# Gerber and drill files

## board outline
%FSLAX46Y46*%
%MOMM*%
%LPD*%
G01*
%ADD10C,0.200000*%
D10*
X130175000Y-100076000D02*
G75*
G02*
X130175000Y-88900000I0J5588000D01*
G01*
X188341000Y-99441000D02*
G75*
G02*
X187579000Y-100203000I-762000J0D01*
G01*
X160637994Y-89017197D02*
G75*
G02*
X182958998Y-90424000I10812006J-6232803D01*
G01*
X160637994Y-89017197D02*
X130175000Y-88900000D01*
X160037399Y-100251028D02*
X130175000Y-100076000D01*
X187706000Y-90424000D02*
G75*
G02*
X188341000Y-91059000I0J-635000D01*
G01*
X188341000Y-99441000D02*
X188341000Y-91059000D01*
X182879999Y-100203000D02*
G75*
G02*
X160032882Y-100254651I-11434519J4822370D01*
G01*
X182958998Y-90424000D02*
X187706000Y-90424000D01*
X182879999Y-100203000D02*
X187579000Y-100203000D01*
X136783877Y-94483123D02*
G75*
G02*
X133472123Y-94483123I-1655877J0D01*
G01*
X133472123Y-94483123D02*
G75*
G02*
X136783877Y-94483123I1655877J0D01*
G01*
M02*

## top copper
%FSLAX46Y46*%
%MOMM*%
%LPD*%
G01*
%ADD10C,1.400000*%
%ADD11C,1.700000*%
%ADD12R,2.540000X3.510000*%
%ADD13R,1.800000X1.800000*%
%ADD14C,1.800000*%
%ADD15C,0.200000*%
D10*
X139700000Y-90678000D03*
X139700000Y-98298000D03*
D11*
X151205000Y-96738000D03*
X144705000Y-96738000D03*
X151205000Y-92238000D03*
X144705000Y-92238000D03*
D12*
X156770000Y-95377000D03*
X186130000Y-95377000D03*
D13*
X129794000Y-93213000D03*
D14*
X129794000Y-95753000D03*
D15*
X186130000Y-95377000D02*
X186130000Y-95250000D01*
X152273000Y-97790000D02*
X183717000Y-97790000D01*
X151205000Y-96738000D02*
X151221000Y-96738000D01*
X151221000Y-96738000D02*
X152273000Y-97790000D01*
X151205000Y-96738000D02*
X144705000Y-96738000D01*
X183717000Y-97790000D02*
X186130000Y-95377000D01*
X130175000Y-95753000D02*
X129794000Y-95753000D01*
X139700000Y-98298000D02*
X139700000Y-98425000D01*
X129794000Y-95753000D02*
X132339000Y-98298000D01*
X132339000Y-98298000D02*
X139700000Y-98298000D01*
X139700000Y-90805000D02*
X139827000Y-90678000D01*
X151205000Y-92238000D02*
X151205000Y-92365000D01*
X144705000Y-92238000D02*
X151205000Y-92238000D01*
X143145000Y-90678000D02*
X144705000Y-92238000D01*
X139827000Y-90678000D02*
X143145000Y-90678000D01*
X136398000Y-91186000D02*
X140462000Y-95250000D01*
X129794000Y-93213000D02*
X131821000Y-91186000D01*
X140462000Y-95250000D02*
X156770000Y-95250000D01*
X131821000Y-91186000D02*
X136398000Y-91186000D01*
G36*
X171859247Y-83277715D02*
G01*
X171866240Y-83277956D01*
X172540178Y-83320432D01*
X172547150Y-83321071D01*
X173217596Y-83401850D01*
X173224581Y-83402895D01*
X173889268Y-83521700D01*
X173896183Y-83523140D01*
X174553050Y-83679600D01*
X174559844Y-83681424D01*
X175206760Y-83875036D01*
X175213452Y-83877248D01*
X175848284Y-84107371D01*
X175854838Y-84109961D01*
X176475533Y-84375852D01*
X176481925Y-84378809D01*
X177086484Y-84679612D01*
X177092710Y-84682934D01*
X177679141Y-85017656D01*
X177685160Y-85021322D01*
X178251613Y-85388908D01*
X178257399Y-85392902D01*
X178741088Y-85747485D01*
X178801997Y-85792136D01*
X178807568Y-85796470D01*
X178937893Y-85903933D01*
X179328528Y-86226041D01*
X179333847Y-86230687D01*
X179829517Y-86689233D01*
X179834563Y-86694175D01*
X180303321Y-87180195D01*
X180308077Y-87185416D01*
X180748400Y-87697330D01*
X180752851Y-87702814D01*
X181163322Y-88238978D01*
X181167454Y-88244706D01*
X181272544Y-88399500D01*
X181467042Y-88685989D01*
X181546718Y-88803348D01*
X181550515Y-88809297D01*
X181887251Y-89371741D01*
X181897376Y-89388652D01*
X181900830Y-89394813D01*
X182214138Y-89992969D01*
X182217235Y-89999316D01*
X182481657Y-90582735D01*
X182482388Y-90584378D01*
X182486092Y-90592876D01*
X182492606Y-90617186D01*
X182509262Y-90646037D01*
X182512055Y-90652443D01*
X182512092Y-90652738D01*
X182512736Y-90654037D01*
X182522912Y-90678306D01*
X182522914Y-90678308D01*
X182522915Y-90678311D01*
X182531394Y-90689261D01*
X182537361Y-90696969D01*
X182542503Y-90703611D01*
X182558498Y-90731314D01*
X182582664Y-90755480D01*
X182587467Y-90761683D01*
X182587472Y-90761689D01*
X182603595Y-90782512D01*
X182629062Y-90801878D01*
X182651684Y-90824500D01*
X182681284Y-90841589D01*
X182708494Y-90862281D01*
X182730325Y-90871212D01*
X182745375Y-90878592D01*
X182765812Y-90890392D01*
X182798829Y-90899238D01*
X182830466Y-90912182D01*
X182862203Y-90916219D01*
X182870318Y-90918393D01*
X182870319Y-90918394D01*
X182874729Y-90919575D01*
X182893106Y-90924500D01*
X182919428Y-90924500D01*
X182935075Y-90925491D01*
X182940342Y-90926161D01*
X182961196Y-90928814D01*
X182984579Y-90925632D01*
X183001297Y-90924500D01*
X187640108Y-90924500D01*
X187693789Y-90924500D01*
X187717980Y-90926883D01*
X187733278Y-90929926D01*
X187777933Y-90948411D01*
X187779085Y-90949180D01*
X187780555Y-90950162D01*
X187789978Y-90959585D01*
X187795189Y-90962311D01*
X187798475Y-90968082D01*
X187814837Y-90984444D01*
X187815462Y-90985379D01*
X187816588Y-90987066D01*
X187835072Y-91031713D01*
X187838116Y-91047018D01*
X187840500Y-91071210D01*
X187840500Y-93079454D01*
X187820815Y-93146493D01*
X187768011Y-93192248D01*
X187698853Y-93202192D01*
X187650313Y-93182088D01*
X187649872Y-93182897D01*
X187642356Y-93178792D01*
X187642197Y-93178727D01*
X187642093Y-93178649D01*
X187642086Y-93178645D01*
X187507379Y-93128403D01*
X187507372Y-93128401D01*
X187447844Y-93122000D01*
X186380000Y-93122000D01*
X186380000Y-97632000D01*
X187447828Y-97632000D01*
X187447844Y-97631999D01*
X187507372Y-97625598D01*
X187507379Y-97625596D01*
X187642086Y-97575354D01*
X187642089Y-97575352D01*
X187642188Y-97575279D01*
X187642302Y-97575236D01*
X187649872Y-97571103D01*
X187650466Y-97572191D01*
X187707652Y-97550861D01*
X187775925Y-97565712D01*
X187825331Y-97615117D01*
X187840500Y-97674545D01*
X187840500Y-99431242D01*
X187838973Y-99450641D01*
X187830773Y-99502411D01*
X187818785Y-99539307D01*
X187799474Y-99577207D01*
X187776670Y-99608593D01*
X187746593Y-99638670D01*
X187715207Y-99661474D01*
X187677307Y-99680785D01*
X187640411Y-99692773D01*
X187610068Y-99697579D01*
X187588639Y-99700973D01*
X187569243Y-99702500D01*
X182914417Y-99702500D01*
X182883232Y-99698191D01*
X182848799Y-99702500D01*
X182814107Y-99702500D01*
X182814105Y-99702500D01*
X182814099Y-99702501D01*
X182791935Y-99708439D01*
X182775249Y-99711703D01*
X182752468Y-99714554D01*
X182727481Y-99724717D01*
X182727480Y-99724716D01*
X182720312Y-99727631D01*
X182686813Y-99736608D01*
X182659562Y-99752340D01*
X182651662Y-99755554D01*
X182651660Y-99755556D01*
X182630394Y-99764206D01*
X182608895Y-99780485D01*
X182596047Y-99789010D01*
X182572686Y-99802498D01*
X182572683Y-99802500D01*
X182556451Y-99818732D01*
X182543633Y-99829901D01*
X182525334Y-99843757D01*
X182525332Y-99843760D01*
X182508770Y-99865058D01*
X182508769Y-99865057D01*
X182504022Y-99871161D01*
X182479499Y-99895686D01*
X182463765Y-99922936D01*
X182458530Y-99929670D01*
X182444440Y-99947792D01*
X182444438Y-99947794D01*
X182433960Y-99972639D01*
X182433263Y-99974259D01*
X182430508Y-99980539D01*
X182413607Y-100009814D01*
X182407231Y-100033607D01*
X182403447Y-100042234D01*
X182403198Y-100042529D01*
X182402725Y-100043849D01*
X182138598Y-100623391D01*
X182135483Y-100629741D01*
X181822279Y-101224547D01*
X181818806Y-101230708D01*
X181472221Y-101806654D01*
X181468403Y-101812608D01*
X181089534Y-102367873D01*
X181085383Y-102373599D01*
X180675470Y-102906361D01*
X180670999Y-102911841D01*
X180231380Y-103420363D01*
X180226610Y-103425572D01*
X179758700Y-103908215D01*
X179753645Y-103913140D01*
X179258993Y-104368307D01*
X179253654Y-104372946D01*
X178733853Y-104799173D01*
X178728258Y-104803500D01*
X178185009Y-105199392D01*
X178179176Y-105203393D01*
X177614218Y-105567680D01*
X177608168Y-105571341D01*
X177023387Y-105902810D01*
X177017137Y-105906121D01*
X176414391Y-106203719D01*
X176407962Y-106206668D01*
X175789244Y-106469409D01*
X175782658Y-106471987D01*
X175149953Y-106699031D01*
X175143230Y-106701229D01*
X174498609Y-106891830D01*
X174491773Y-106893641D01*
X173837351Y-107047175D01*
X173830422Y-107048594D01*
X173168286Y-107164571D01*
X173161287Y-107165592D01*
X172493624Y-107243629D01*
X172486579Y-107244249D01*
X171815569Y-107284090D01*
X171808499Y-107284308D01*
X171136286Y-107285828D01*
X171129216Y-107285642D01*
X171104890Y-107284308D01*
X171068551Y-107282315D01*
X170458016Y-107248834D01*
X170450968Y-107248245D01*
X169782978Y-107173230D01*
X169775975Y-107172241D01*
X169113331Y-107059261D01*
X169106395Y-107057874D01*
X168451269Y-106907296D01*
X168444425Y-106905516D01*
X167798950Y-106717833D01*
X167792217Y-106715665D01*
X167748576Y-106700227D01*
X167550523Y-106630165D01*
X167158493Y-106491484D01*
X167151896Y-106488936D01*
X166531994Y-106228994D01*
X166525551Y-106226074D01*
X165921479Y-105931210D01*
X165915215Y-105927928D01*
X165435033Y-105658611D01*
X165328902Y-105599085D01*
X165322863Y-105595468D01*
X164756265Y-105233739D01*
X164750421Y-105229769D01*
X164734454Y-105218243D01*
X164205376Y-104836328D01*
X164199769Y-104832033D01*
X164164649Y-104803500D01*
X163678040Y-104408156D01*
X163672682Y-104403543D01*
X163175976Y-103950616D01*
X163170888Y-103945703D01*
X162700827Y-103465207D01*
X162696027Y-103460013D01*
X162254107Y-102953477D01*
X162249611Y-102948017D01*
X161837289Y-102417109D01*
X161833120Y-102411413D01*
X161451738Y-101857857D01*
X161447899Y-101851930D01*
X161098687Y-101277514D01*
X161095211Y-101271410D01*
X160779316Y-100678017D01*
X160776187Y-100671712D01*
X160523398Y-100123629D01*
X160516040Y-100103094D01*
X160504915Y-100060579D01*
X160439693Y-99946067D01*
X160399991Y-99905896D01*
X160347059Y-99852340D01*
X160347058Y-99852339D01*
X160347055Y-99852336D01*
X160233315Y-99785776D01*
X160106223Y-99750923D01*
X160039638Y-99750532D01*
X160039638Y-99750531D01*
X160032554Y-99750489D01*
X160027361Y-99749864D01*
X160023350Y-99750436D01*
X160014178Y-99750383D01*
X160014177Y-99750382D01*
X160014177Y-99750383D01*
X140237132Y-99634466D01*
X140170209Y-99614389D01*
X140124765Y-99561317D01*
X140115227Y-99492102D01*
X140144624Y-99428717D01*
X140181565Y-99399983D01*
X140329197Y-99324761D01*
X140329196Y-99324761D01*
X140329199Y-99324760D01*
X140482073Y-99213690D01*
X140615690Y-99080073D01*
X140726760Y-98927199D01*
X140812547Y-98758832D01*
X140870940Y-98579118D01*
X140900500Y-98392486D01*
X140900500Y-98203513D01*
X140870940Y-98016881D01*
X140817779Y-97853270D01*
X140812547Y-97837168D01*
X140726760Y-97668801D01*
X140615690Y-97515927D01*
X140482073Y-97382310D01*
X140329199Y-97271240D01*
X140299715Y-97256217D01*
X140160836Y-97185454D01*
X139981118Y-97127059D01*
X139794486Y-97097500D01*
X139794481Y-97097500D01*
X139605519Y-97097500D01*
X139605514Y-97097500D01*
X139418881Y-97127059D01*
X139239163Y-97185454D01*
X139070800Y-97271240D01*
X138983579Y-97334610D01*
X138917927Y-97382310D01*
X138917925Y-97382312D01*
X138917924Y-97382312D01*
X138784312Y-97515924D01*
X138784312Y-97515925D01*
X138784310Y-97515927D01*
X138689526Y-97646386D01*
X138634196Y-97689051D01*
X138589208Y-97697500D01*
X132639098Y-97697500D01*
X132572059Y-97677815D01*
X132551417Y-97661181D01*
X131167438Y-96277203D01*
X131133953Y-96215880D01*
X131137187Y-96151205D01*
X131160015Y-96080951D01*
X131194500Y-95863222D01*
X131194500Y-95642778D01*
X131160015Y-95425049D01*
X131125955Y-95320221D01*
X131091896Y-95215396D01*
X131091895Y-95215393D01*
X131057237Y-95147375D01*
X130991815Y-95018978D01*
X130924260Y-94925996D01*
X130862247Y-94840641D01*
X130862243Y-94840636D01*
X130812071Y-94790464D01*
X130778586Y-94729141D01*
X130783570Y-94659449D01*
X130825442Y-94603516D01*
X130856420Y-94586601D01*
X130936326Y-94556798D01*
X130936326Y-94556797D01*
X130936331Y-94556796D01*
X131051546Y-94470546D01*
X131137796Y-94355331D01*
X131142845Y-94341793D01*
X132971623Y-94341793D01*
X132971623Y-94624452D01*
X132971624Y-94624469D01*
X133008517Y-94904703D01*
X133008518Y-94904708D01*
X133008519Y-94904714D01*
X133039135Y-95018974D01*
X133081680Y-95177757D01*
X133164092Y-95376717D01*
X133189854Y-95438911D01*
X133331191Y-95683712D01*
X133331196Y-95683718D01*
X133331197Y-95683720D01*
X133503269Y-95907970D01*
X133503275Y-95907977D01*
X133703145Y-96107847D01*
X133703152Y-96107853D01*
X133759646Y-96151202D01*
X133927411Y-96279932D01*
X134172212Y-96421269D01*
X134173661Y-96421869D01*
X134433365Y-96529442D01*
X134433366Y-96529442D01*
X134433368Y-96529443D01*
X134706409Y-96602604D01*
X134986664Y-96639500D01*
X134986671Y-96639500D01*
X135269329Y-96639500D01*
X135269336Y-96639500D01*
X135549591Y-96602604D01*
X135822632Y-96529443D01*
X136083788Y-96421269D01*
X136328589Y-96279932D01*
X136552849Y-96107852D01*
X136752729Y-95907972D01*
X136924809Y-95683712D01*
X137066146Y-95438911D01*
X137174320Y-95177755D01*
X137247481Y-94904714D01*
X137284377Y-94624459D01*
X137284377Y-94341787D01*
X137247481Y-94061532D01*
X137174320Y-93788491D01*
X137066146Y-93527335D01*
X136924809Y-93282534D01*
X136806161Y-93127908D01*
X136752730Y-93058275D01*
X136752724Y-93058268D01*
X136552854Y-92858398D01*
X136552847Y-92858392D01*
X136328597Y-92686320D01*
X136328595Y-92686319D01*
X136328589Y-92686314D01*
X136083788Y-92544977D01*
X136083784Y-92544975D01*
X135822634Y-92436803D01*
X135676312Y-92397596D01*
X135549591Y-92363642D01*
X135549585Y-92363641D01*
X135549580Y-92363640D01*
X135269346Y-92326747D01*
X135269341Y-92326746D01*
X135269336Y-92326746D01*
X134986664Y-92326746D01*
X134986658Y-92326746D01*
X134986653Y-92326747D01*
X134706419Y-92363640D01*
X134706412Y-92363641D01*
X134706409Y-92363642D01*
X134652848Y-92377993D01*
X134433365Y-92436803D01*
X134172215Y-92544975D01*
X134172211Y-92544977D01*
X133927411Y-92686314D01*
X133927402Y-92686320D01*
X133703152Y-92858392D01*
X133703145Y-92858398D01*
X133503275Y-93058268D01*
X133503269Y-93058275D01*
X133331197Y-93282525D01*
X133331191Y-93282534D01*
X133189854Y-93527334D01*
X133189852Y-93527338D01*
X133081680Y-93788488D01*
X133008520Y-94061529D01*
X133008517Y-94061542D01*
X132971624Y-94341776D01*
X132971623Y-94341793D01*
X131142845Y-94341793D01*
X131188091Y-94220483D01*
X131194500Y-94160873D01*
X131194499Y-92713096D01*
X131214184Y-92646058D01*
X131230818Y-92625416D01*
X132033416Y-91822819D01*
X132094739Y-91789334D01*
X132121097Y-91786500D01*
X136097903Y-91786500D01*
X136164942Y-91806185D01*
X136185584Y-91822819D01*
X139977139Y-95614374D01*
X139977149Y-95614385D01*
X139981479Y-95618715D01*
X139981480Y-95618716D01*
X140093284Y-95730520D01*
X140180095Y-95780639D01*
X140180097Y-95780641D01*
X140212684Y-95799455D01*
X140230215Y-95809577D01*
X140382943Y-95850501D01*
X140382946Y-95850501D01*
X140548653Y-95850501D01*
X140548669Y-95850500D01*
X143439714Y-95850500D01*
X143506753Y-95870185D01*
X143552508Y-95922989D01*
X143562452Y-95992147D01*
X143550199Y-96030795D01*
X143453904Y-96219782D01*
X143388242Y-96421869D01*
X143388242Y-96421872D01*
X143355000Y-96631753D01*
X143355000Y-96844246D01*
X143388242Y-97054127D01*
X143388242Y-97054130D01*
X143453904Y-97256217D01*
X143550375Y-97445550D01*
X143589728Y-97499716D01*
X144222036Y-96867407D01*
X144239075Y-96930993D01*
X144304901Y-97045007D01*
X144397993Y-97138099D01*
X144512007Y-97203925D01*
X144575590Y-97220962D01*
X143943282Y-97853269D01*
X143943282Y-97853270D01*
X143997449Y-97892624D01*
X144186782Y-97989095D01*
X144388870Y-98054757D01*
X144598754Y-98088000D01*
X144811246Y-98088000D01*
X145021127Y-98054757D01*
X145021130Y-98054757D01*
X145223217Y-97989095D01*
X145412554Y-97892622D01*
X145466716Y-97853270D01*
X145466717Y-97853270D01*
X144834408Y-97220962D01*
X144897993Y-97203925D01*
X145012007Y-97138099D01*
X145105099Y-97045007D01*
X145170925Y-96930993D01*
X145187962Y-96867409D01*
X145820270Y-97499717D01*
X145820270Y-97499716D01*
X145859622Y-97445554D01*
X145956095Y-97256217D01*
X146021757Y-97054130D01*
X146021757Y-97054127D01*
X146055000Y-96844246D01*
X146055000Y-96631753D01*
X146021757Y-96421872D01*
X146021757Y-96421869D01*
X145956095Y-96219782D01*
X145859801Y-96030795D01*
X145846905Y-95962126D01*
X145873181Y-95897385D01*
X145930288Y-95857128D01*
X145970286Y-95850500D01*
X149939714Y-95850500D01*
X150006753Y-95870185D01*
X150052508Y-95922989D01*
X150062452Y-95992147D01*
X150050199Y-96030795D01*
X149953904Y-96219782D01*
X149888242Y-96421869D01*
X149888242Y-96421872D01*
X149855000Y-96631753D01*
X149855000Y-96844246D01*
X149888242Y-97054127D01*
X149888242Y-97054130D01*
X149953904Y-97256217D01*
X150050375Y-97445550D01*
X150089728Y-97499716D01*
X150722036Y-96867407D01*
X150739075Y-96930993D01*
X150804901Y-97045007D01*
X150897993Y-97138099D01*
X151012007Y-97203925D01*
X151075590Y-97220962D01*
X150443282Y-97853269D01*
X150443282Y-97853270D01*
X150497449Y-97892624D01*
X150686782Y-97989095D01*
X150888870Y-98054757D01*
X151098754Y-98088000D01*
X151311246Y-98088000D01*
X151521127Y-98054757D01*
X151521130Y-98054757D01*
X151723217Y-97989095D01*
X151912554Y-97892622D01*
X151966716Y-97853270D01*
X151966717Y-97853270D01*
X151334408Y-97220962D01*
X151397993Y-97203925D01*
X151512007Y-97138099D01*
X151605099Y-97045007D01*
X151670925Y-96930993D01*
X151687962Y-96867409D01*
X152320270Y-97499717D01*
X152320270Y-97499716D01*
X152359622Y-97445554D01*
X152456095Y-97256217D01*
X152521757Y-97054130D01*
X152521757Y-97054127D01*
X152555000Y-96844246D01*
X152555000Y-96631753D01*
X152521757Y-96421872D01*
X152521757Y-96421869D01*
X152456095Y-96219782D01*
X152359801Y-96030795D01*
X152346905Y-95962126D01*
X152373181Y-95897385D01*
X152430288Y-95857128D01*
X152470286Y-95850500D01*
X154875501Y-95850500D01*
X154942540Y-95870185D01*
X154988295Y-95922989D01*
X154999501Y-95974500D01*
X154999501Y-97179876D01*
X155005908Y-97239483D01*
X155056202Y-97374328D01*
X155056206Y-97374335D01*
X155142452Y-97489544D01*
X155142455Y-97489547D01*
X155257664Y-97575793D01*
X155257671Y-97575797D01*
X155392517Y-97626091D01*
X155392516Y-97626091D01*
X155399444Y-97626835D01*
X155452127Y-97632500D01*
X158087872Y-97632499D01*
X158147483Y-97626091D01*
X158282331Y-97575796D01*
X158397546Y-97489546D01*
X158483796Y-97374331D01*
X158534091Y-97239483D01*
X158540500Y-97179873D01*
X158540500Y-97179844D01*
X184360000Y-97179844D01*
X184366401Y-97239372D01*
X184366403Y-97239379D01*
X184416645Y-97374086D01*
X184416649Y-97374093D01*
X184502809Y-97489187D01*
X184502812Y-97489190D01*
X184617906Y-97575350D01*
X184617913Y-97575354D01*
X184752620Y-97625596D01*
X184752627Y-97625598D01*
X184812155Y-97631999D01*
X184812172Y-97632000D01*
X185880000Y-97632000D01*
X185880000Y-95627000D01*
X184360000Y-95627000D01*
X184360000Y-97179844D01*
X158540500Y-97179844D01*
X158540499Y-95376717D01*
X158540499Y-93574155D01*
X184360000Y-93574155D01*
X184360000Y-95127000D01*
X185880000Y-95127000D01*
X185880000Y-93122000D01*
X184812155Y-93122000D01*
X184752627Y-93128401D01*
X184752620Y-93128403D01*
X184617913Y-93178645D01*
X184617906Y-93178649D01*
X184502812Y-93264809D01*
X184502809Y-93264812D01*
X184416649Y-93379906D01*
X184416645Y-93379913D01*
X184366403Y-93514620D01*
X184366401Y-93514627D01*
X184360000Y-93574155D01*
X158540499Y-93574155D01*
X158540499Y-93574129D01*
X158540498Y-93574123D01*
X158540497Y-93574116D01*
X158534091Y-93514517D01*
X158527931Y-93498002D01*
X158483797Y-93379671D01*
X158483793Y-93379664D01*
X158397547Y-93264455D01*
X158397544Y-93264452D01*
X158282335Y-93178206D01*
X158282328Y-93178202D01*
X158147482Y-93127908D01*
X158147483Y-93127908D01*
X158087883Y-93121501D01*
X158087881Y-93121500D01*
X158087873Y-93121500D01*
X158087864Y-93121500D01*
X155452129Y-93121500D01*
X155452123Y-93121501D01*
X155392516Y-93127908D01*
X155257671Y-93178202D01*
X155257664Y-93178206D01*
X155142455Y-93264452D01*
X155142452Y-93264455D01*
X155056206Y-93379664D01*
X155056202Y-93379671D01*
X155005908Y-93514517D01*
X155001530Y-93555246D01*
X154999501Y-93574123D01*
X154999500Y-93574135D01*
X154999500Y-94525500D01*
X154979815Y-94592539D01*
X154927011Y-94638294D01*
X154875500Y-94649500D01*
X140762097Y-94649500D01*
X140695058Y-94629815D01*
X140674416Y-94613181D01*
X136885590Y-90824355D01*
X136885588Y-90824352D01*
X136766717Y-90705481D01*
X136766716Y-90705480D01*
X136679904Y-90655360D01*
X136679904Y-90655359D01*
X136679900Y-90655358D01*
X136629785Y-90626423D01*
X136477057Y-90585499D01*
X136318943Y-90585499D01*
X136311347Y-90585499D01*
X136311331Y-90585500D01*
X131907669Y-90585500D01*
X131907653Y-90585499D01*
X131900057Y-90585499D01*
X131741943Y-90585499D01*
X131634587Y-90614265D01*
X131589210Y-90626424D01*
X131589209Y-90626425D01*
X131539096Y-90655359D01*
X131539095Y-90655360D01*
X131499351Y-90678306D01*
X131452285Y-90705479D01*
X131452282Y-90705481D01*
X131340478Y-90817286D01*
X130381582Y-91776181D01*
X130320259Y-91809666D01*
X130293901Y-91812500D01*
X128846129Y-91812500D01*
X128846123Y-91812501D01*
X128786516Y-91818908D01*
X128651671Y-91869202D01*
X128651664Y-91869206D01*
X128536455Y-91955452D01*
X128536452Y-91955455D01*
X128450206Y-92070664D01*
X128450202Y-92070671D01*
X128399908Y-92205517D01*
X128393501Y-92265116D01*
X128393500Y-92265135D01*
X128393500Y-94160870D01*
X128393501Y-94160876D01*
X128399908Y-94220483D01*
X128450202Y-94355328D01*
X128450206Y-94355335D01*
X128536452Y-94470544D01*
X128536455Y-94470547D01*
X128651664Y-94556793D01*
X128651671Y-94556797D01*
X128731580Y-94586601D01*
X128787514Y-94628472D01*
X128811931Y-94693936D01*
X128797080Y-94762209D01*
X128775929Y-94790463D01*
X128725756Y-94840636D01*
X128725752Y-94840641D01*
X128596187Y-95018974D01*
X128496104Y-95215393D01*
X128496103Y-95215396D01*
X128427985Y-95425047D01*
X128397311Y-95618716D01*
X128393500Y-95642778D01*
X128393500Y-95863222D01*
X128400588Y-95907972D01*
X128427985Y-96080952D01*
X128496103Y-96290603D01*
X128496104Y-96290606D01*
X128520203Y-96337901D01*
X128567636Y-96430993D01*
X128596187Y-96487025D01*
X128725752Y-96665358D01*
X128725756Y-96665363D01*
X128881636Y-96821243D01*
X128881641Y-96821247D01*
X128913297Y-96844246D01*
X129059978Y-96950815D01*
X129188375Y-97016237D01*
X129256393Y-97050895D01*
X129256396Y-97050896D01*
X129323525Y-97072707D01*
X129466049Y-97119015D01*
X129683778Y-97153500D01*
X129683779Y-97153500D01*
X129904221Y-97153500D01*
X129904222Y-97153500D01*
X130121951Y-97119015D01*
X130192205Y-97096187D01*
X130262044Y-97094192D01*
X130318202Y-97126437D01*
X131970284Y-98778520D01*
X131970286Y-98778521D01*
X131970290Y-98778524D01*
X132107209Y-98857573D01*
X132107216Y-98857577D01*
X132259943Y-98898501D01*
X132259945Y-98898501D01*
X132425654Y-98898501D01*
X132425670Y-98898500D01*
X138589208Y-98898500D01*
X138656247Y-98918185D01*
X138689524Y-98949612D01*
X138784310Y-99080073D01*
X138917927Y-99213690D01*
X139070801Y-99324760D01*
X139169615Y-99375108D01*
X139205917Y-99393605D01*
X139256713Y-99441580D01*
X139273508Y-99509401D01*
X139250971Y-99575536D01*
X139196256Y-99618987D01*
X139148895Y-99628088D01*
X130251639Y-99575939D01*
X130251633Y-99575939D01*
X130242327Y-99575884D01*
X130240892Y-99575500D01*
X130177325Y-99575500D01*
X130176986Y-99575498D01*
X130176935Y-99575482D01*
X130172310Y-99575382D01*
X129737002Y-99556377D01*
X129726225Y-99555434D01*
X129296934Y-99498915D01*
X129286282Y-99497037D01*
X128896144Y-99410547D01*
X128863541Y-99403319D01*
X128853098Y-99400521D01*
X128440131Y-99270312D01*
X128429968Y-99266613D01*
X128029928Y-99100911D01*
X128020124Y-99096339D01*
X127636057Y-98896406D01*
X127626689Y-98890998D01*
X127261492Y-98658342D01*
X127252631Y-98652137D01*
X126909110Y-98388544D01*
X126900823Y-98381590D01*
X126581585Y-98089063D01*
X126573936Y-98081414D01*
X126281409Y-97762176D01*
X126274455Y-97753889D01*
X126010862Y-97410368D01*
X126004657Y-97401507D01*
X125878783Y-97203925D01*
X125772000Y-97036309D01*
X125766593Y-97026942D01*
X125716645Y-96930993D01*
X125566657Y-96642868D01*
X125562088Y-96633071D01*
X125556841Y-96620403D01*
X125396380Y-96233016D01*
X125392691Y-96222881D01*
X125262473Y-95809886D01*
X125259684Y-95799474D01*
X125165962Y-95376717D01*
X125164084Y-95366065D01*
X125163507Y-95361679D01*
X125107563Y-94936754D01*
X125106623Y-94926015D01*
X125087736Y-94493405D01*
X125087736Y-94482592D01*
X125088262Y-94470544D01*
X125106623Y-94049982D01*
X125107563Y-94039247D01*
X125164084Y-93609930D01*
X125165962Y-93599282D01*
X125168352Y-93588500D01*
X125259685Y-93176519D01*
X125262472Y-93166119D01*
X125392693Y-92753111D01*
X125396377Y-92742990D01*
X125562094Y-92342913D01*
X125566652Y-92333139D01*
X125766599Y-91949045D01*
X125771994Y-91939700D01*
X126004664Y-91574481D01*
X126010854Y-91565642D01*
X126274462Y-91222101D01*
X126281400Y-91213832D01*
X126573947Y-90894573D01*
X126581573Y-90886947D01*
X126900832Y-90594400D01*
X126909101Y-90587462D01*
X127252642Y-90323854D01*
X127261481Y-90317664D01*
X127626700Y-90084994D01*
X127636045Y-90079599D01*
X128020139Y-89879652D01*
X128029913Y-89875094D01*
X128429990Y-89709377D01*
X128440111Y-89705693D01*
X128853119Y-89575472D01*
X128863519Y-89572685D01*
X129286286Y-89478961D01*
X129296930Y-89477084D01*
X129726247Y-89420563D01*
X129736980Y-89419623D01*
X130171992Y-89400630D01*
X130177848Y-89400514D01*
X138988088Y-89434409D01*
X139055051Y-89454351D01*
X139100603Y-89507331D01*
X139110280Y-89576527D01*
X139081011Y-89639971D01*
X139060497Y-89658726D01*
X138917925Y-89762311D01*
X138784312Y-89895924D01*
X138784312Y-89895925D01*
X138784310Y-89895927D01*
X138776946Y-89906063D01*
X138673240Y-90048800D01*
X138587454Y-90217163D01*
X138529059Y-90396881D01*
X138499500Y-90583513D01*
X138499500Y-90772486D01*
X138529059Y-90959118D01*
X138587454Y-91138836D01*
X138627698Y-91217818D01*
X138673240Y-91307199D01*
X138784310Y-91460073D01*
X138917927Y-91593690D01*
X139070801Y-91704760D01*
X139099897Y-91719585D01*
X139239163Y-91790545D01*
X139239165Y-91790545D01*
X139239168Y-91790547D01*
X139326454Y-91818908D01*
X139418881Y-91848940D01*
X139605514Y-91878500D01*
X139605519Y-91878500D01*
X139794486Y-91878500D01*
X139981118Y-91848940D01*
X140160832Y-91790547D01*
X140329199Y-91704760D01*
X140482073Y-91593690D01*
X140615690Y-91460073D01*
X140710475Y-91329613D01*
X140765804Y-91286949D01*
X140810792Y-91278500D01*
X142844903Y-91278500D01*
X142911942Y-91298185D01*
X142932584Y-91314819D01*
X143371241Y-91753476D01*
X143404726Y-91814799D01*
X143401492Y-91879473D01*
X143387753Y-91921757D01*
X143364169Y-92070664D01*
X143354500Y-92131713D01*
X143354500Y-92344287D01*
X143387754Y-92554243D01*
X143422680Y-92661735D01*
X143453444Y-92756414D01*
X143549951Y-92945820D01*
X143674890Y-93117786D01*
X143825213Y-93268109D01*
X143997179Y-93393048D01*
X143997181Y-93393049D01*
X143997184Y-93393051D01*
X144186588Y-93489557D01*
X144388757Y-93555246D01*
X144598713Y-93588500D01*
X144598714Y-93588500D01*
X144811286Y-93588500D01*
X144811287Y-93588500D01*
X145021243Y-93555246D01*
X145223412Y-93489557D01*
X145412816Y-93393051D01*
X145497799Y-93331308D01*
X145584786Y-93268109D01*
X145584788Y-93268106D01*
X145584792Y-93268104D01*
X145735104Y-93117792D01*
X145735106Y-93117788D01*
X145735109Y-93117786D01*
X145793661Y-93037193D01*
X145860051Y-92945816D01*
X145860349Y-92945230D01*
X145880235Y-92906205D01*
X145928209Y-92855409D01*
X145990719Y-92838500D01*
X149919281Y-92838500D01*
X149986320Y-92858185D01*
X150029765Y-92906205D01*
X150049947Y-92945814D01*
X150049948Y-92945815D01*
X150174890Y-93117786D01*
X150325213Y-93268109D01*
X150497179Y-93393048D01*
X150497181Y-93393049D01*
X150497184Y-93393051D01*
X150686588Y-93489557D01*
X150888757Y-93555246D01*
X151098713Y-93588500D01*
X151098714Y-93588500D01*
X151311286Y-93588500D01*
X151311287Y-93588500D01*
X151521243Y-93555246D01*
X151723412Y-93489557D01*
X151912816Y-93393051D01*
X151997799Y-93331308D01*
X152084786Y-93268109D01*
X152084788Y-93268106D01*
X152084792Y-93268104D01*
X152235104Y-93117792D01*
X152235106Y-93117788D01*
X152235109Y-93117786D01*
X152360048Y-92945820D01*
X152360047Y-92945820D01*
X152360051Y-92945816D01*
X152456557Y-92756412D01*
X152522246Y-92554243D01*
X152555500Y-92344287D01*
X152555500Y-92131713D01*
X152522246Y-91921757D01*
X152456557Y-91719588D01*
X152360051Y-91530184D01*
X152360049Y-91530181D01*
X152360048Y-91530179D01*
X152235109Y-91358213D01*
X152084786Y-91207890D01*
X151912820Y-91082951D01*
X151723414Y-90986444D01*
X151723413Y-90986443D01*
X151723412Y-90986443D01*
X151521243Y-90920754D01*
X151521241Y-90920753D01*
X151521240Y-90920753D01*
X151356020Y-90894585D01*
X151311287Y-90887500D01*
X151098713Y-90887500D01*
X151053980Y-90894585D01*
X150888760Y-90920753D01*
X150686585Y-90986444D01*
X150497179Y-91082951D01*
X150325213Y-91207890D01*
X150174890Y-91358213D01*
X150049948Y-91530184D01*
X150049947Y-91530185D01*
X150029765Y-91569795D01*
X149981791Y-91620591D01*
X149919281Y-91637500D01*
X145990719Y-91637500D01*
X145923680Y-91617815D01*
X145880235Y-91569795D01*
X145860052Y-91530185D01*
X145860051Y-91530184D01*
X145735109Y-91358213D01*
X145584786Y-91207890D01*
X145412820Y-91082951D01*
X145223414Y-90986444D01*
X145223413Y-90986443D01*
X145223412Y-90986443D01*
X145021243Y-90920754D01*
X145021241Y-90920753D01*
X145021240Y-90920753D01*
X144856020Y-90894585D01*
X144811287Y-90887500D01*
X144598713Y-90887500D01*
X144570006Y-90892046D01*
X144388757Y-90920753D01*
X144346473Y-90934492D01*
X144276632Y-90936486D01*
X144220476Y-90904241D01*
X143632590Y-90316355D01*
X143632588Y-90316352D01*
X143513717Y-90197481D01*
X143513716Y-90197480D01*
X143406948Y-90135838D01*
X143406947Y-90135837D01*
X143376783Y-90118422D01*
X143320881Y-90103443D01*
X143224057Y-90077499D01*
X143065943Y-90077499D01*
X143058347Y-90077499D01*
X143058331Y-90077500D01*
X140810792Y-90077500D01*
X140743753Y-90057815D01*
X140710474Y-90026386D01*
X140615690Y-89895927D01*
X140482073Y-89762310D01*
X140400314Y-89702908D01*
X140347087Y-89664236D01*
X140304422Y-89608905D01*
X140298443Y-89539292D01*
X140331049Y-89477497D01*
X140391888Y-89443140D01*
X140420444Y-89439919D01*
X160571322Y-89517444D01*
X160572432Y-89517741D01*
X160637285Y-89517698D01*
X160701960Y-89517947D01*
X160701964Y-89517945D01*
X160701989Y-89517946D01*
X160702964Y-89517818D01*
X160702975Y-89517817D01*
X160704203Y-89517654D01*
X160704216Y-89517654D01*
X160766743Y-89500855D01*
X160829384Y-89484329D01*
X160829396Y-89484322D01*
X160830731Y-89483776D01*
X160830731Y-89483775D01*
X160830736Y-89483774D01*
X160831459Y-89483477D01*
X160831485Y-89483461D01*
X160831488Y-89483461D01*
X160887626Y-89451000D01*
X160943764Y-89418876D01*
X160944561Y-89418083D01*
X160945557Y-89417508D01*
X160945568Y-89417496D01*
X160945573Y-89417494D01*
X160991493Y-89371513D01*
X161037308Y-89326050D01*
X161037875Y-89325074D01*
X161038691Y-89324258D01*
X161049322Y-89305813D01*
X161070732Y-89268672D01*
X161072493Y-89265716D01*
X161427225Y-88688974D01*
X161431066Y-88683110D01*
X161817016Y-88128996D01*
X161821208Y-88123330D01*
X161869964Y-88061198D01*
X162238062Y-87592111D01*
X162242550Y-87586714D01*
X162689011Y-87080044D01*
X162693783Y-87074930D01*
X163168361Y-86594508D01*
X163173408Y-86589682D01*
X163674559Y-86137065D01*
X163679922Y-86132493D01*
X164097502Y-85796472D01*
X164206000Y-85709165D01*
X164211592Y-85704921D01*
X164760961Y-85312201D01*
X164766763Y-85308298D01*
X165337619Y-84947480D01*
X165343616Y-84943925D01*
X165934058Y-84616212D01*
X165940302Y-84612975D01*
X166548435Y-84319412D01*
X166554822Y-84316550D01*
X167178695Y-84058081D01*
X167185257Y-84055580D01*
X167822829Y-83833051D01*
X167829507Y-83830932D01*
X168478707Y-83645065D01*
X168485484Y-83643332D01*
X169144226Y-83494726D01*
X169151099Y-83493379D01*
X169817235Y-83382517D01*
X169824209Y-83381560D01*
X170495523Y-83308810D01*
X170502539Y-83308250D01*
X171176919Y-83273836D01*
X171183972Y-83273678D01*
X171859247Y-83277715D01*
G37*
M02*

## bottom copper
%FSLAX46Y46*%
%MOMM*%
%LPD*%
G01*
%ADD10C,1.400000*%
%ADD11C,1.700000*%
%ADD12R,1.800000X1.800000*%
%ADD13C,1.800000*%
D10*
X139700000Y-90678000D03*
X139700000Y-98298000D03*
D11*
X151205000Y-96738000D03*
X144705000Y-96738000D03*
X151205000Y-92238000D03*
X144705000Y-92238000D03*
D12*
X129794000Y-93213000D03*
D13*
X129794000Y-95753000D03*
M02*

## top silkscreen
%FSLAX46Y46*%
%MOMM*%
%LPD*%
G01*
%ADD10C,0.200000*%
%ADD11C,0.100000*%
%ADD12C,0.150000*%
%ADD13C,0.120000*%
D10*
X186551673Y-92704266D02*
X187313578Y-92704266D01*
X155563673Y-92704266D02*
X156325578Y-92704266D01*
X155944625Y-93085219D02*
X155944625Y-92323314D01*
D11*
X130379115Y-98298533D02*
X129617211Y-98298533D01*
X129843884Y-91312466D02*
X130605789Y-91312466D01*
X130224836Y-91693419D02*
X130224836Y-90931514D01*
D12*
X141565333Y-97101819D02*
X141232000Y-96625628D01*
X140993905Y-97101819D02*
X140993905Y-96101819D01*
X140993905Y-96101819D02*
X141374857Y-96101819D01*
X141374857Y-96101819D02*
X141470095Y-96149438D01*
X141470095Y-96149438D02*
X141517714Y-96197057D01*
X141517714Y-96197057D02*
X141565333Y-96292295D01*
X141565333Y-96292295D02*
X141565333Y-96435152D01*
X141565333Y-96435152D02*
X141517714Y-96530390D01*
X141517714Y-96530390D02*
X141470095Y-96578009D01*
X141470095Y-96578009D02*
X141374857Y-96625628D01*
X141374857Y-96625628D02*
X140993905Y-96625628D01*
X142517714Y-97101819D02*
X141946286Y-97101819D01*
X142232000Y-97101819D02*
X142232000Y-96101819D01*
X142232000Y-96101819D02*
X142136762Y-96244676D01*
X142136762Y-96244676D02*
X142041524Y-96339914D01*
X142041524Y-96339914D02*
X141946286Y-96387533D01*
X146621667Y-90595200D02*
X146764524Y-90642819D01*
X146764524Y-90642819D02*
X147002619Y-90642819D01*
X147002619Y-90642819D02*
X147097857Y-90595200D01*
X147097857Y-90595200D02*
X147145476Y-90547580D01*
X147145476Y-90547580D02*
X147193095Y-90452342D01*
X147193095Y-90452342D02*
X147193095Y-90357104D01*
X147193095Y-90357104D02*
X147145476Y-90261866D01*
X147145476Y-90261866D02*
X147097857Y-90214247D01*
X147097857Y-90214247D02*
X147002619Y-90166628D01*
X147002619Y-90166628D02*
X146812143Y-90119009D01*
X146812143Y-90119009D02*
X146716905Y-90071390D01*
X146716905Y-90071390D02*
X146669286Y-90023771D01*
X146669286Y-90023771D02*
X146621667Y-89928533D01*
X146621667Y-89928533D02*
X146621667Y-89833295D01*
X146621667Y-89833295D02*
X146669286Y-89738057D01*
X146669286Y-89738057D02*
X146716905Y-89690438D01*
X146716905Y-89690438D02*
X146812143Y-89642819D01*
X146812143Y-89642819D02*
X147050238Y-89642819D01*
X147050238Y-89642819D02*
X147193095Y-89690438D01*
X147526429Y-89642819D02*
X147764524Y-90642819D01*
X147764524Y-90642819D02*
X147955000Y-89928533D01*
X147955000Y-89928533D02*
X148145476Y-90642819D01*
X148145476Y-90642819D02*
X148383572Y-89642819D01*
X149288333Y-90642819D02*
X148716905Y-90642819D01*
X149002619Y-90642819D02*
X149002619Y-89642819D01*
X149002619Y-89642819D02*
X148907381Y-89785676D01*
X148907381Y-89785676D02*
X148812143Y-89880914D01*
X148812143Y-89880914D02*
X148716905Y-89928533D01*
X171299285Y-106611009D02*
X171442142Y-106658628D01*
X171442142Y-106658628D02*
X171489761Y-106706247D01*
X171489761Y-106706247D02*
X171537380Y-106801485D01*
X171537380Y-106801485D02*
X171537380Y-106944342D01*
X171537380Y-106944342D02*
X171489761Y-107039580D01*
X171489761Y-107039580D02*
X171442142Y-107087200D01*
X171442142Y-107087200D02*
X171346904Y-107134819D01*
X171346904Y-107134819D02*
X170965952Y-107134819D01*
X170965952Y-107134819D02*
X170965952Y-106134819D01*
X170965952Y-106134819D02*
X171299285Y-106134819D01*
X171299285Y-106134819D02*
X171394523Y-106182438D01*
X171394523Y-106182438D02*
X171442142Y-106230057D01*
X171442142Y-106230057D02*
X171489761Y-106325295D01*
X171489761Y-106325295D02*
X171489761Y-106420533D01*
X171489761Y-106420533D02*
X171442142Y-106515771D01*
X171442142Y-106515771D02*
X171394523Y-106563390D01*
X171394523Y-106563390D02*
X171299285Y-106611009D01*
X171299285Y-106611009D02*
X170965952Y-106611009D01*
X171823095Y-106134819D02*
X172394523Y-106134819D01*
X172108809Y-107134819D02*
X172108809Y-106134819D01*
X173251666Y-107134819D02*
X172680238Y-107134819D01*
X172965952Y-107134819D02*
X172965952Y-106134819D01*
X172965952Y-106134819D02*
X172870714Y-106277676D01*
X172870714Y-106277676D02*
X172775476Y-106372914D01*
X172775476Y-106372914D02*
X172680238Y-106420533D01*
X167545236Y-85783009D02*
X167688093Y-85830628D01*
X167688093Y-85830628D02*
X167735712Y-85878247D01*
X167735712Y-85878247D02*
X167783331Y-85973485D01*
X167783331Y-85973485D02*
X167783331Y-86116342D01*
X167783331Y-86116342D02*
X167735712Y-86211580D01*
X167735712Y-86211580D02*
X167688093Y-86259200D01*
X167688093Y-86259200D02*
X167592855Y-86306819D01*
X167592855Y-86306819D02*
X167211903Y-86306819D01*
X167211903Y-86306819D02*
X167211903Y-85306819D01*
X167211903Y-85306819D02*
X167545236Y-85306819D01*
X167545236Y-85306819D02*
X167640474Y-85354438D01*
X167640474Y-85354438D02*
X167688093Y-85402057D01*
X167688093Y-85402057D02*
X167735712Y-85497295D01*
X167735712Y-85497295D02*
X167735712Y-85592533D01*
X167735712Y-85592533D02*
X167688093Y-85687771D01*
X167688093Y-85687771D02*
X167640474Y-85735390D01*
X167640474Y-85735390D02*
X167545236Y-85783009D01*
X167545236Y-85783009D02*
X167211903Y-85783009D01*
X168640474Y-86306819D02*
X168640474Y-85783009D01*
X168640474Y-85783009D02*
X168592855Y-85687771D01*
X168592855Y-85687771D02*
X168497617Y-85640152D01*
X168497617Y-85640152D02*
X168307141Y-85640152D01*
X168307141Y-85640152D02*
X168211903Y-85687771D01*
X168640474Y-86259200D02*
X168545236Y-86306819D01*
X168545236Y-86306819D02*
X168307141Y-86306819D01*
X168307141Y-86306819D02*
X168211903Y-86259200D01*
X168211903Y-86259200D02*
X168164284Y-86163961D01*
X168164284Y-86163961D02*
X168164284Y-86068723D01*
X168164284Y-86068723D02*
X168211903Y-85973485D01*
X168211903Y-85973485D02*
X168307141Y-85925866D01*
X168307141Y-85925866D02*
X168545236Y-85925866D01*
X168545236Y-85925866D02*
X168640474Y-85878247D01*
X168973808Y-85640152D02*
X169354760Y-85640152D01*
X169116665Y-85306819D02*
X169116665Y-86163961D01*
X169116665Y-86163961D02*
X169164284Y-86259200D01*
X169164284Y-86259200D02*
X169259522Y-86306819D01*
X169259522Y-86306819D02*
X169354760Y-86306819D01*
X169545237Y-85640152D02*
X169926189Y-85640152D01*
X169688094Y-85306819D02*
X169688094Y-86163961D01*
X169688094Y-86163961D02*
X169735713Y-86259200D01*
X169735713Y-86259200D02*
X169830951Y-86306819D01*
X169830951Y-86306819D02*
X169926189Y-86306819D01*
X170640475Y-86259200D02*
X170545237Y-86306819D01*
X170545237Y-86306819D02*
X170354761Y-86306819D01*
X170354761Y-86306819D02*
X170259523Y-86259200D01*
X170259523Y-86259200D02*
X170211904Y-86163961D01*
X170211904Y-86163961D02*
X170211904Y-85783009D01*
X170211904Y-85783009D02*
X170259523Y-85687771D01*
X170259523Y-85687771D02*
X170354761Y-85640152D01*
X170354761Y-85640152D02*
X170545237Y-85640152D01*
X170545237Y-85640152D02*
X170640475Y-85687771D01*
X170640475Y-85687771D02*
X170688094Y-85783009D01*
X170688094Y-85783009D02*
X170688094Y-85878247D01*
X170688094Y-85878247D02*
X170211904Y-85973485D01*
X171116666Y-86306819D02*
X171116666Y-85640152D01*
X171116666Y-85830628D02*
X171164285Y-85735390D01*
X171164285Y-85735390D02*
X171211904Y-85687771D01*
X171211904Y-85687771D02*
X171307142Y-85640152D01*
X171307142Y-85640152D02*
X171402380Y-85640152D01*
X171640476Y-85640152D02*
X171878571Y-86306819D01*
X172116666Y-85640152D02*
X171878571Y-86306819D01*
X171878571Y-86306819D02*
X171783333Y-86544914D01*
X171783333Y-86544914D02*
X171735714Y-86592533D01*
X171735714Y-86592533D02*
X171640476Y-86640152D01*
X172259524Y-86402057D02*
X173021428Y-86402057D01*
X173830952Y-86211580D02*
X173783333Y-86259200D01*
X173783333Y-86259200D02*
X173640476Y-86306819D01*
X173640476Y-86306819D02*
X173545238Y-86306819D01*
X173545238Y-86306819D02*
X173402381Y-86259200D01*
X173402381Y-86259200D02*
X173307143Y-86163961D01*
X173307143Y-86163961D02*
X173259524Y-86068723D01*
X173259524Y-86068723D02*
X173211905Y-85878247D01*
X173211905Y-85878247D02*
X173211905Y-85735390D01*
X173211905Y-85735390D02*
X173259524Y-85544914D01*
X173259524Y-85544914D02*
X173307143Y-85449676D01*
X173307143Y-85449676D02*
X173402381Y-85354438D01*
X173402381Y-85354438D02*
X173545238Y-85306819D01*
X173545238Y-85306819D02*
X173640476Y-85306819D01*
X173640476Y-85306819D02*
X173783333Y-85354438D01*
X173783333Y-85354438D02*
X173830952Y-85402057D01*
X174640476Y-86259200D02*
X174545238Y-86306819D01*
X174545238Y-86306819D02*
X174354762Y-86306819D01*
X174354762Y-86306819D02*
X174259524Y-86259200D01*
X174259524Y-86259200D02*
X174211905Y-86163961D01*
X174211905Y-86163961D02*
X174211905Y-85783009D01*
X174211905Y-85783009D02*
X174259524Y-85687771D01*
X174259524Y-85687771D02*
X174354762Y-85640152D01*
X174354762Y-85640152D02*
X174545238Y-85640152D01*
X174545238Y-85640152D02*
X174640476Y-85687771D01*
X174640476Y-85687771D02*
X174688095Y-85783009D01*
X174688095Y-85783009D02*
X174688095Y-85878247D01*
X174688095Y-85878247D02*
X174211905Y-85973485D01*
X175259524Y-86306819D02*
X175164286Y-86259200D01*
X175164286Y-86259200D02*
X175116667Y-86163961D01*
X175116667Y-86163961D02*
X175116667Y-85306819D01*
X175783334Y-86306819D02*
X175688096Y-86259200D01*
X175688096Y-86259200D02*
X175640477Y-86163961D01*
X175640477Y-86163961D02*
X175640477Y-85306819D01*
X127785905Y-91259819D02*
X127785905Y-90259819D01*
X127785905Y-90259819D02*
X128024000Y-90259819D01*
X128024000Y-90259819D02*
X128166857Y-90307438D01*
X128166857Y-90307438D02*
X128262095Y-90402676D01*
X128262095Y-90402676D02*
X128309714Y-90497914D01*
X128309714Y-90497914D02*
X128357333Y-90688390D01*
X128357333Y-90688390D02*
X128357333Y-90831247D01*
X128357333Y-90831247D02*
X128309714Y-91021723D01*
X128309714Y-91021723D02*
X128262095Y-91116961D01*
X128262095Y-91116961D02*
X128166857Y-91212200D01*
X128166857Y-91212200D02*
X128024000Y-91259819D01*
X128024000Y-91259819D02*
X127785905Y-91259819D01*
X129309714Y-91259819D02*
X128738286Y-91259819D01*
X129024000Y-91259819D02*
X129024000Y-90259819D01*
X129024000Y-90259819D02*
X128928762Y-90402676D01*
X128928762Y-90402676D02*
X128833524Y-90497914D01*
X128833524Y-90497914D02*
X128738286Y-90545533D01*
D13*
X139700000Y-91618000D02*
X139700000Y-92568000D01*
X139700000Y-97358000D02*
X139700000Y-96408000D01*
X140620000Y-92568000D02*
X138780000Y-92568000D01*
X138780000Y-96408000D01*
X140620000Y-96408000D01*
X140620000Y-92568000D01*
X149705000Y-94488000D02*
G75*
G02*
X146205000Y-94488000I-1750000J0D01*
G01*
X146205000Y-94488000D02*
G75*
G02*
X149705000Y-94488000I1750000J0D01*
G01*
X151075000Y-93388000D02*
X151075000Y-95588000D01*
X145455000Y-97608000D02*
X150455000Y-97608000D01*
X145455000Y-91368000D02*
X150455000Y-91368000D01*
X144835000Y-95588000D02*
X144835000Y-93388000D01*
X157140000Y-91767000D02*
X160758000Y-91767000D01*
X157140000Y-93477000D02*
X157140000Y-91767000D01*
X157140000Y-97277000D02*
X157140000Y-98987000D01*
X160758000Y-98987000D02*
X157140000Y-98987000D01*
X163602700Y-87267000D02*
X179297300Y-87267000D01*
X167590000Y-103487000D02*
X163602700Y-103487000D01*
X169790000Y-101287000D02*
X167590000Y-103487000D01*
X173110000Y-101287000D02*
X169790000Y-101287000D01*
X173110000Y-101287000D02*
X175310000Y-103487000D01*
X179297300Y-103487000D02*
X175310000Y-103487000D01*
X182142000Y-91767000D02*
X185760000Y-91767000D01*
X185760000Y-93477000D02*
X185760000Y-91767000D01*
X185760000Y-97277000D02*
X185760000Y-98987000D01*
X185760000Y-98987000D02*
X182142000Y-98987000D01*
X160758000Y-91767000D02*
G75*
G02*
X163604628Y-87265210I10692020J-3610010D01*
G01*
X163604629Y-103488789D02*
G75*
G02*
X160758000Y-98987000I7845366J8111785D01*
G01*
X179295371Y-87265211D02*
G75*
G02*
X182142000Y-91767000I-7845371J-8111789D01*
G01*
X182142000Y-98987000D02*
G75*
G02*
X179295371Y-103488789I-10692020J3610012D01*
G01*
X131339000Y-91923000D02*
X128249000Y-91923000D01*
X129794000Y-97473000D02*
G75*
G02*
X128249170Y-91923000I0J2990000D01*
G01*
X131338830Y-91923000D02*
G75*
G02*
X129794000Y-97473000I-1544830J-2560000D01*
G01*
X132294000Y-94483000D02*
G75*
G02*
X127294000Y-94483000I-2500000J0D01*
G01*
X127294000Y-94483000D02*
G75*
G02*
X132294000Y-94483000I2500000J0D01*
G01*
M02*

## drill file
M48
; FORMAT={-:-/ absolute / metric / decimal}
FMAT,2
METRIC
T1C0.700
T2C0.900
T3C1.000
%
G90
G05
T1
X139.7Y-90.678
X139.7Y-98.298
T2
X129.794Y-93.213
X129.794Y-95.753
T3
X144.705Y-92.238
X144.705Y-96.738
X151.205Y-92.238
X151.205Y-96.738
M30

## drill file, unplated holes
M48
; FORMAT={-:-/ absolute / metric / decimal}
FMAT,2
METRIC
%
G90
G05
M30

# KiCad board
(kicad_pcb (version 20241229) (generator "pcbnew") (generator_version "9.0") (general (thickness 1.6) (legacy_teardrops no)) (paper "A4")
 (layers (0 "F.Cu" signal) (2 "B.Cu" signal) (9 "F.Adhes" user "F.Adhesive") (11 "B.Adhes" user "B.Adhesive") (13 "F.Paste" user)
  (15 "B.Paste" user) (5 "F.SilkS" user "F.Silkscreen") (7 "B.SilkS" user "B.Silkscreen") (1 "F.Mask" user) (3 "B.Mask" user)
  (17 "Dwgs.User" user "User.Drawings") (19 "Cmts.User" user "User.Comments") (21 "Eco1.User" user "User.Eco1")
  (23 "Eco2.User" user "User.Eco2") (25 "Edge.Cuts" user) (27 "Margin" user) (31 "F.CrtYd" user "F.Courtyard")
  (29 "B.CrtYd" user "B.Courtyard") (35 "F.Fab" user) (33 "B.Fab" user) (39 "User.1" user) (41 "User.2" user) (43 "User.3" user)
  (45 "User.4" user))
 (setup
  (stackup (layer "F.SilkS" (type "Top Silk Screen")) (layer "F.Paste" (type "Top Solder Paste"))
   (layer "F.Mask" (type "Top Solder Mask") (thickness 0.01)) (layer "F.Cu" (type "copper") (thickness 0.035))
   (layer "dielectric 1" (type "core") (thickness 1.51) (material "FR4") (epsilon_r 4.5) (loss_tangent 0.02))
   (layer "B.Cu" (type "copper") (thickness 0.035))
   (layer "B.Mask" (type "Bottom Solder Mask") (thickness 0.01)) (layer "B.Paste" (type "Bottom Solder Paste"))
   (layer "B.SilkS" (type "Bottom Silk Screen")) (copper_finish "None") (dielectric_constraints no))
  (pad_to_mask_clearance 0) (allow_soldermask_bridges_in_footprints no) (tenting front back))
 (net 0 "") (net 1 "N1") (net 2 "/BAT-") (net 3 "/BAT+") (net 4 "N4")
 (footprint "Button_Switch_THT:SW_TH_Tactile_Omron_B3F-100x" (layer "F.Cu") (at 144.705 92.238)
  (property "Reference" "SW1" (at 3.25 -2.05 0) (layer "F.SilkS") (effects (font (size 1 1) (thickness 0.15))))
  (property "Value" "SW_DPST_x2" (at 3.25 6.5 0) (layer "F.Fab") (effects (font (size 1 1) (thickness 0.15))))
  (fp_line (start 0.13 3.35) (end 0.13 1.15) (stroke (width 0.12) (type solid)) (layer "F.SilkS"))
  (fp_line (start 0.75 -0.87) (end 5.75 -0.87) (stroke (width 0.12) (type solid)) (layer "F.SilkS"))
  (fp_line (start 0.75 5.37) (end 5.75 5.37) (stroke (width 0.12) (type solid)) (layer "F.SilkS"))
  (fp_line (start 6.37 1.15) (end 6.37 3.35) (stroke (width 0.12) (type solid)) (layer "F.SilkS"))
  (fp_circle (center 3.25 2.25) (end 5 2.25) (stroke (width 0.12) (type solid)) (fill no) (layer "F.SilkS"))
  (pad "1" thru_hole circle (at 0 0) (size 1.7 1.7) (drill 1) (layers "*.Cu" "*.Mask") (remove_unused_layers no) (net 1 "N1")
   (thermal_bridge_angle 90))
  (pad "1" thru_hole circle (at 6.5 0) (size 1.7 1.7) (drill 1) (layers "*.Cu" "*.Mask") (remove_unused_layers no) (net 1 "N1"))
  (pad "2" thru_hole circle (at 0 4.5) (size 1.7 1.7) (drill 1) (layers "*.Cu" "*.Mask") (remove_unused_layers no) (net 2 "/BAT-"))
  (pad "2" thru_hole circle (at 6.5 4.5) (size 1.7 1.7) (drill 1) (layers "*.Cu" "*.Mask") (remove_unused_layers no) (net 2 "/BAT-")))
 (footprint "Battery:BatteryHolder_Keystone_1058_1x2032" (layer "F.Cu") (at 171.45 95.377)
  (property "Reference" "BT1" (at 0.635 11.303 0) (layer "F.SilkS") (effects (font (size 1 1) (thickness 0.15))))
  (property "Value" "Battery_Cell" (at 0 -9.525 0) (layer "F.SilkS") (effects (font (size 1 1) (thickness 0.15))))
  (fp_line (start -14.31 -3.61) (end -10.692 -3.61) (stroke (width 0.12) (type solid)) (layer "F.SilkS"))
  (fp_line (start -14.31 -1.9) (end -14.31 -3.61) (stroke (width 0.12) (type solid)) (layer "F.SilkS"))
  (fp_line (start -14.31 1.9) (end -14.31 3.61) (stroke (width 0.12) (type solid)) (layer "F.SilkS"))
  (fp_line (start -10.692 3.61) (end -14.31 3.61) (stroke (width 0.12) (type solid)) (layer "F.SilkS"))
  (fp_line (start -7.8473 -8.11) (end 7.8473 -8.11) (stroke (width 0.12) (type solid)) (layer "F.SilkS"))
  (fp_line (start -3.86 8.11) (end -7.8473 8.11) (stroke (width 0.12) (type solid)) (layer "F.SilkS"))
  (fp_line (start -1.66 5.91) (end -3.86 8.11) (stroke (width 0.12) (type solid)) (layer "F.SilkS"))
  (fp_line (start 1.66 5.91) (end -1.66 5.91) (stroke (width 0.12) (type solid)) (layer "F.SilkS"))
  (fp_line (start 1.66 5.91) (end 3.86 8.11) (stroke (width 0.12) (type solid)) (layer "F.SilkS"))
  (fp_line (start 7.8473 8.11) (end 3.86 8.11) (stroke (width 0.12) (type solid)) (layer "F.SilkS"))
  (fp_line (start 10.692 -3.61) (end 14.31 -3.61) (stroke (width 0.12) (type solid)) (layer "F.SilkS"))
  (fp_line (start 14.31 -1.9) (end 14.31 -3.61) (stroke (width 0.12) (type solid)) (layer "F.SilkS"))
  (fp_line (start 14.31 1.9) (end 14.31 3.61) (stroke (width 0.12) (type solid)) (layer "F.SilkS"))
  (fp_line (start 14.31 3.61) (end 10.692 3.61) (stroke (width 0.12) (type solid)) (layer "F.SilkS"))
  (fp_arc (start -10.692 -3.61) (mid -9.538084 -6.031244) (end -7.845371 -8.111789) (stroke (width 0.12) (type solid)) (layer "F.SilkS"))
  (fp_arc (start -7.845371 8.111789) (mid -9.538085 6.031244) (end -10.692 3.61) (stroke (width 0.12) (type solid)) (layer "F.SilkS"))
  (fp_arc (start 7.845371 -8.111789) (mid 9.538085 -6.031244) (end 10.692 -3.61) (stroke (width 0.12) (type solid)) (layer "F.SilkS"))
  (fp_arc (start 10.692 3.61) (mid 9.538084 6.031244) (end 7.845371 8.111789) (stroke (width 0.12) (type solid)) (layer "F.SilkS"))
  (pad "1" smd rect (at -14.68 0) (size 2.54 3.51) (layers "F.Cu" "F.Mask" "F.Paste") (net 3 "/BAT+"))
  (pad "2" smd rect (at 14.68 0) (size 2.54 3.51) (layers "F.Cu" "F.Mask" "F.Paste") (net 2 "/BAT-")))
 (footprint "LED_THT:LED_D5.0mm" (layer "F.Cu") (at 129.794 93.213 -90)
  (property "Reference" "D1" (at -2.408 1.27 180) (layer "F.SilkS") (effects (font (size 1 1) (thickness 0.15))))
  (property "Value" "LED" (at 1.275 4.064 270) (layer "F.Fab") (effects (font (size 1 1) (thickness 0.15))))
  (fp_line (start -1.29 -1.545) (end -1.29 1.545) (stroke (width 0.12) (type solid)) (layer "F.SilkS"))
  (fp_arc (start 4.26 0) (mid 2.071779 2.880495) (end -1.29 1.54483) (stroke (width 0.12) (type solid)) (layer "F.SilkS"))
  (fp_arc (start -1.29 -1.54483) (mid 2.071779 -2.880495) (end 4.26 0) (stroke (width 0.12) (type solid)) (layer "F.SilkS"))
  (fp_circle (center 1.27 0) (end 3.77 0) (stroke (width 0.12) (type solid)) (fill no) (layer "F.SilkS"))
  (pad "1" thru_hole rect (at 0 0 270) (size 1.8 1.8) (drill 0.9) (layers "*.Cu" "*.Mask") (remove_unused_layers no) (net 3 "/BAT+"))
  (pad "2" thru_hole circle (at 2.54 0 270) (size 1.8 1.8) (drill 0.9) (layers "*.Cu" "*.Mask") (remove_unused_layers no) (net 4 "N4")))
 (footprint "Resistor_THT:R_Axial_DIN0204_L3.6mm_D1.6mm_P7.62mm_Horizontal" (layer "F.Cu") (at 139.7 90.678 -90)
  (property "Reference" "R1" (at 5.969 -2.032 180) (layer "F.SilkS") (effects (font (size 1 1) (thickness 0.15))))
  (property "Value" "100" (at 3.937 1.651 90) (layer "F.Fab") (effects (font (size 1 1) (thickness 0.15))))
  (fp_line (start 0.94 0) (end 1.89 0) (stroke (width 0.12) (type solid)) (layer "F.SilkS"))
  (fp_line (start 6.68 0) (end 5.73 0) (stroke (width 0.12) (type solid)) (layer "F.SilkS"))
  (fp_rect (start 1.89 -0.92) (end 5.73 0.92) (stroke (width 0.12) (type solid)) (fill no) (layer "F.SilkS"))
  (pad "1" thru_hole circle (at 0 0 270) (size 1.4 1.4) (drill 0.7) (layers "*.Cu" "*.Mask") (remove_unused_layers no) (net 1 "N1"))
  (pad "2" thru_hole circle (at 7.62 0 270) (size 1.4 1.4) (drill 0.7) (layers "*.Cu" "*.Mask") (remove_unused_layers no) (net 4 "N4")))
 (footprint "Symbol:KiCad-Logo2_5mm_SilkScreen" (layer "B.Cu") (at 171.704 90.17 180)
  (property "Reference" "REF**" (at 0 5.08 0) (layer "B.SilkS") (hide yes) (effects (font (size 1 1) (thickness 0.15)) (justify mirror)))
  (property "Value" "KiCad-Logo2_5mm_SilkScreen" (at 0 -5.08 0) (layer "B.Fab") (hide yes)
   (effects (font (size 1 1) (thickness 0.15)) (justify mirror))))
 (gr_arc (start 130.175 100.076) (mid 124.587 94.488) (end 130.175 88.9) (stroke (width 0.2) (type default)) (locked yes)
  (layer "Edge.Cuts"))
 (gr_arc (start 188.341 99.441) (mid 188.117815 99.979815) (end 187.579 100.203) (stroke (width 0.2) (type default)) (locked yes)
  (layer "Edge.Cuts"))
 (gr_arc (start 160.637994 89.017197) (mid 172.234999 82.794837) (end 182.958998 90.424) (stroke (width 0.2) (type default)) (locked yes)
  (layer "Edge.Cuts"))
 (gr_line (start 160.637994 89.017197) (end 130.175 88.9) (stroke (width 0.2) (type default)) (locked yes) (layer "Edge.Cuts"))
 (gr_circle (center 135.128 94.483123) (end 135.255 92.832123) (stroke (width 0.2) (type solid)) (fill no) (locked yes) (layer "Edge.Cuts"))
 (gr_line (start 160.037399 100.251028) (end 130.175 100.076) (stroke (width 0.2) (type default)) (locked yes) (layer "Edge.Cuts"))
 (gr_arc (start 187.706 90.424) (mid 188.155013 90.609987) (end 188.341 91.059) (stroke (width 0.2) (type default)) (locked yes)
  (layer "Edge.Cuts"))
 (gr_line (start 188.341 99.441) (end 188.341 91.059) (stroke (width 0.2) (type default)) (locked yes) (layer "Edge.Cuts"))
 (gr_arc (start 182.879999 100.203) (mid 171.473533 107.790412) (end 160.032877 100.254653) (stroke (width 0.2) (type default)) (locked yes)
  (layer "Edge.Cuts"))
 (gr_line (start 182.958998 90.424) (end 187.706 90.424) (stroke (width 0.2) (type default)) (locked yes) (layer "Edge.Cuts"))
 (gr_line (start 182.879999 100.203) (end 187.579 100.203) (stroke (width 0.2) (type default)) (locked yes) (layer "Edge.Cuts"))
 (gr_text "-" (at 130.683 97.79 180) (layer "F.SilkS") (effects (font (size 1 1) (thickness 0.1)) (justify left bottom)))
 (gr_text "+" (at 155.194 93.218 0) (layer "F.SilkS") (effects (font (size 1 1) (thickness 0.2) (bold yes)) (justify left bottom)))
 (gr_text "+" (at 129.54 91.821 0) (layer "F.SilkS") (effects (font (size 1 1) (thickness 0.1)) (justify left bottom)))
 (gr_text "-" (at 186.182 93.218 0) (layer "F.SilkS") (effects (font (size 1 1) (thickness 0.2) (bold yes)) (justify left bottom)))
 (segment (start 136.398 91.186) (end 140.462 95.25) (width 0.2) (layer "F.Cu") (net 3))
 (segment (start 129.794 93.213) (end 131.821 91.186) (width 0.2) (layer "F.Cu") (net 3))
 (segment (start 140.462 95.25) (end 156.77 95.25) (width 0.2) (layer "F.Cu") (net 3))
 (segment (start 131.821 91.186) (end 136.398 91.186) (width 0.2) (layer "F.Cu") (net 3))
 (segment (start 186.13 95.377) (end 186.13 95.25) (width 0.2) (layer "F.Cu") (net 2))
 (segment (start 152.273 97.79) (end 183.717 97.79) (width 0.2) (layer "F.Cu") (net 2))
 (segment (start 151.205 96.738) (end 151.221 96.738) (width 0.2) (layer "F.Cu") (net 2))
 (segment (start 151.221 96.738) (end 152.273 97.79) (width 0.2) (layer "F.Cu") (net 2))
 (segment (start 151.205 96.738) (end 144.705 96.738) (width 0.2) (layer "F.Cu") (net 2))
 (segment (start 183.717 97.79) (end 186.13 95.377) (width 0.2) (layer "F.Cu") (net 2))
 (segment (start 139.7 90.805) (end 139.827 90.678) (width 0.2) (layer "F.Cu") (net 1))
 (segment (start 151.205 92.238) (end 151.205 92.365) (width 0.2) (layer "F.Cu") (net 1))
 (segment (start 144.705 92.238) (end 151.205 92.238) (width 0.2) (layer "F.Cu") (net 1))
 (segment (start 143.145 90.678) (end 144.705 92.238) (width 0.2) (layer "F.Cu") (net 1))
 (segment (start 139.827 90.678) (end 143.145 90.678) (width 0.2) (layer "F.Cu") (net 1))
 (segment (start 130.175 95.753) (end 129.794 95.753) (width 0.2) (layer "F.Cu") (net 4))
 (segment (start 139.7 98.298) (end 139.7 98.425) (width 0.2) (layer "F.Cu") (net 4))
 (segment (start 129.794 95.753) (end 132.339 98.298) (width 0.2) (layer "F.Cu") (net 4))
 (segment (start 132.339 98.298) (end 139.7 98.298) (width 0.2) (layer "F.Cu") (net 4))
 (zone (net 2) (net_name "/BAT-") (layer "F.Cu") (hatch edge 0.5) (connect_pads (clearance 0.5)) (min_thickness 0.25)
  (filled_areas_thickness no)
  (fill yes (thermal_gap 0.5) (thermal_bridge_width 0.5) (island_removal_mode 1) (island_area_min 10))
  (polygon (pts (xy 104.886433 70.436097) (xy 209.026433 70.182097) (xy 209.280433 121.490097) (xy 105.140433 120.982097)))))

